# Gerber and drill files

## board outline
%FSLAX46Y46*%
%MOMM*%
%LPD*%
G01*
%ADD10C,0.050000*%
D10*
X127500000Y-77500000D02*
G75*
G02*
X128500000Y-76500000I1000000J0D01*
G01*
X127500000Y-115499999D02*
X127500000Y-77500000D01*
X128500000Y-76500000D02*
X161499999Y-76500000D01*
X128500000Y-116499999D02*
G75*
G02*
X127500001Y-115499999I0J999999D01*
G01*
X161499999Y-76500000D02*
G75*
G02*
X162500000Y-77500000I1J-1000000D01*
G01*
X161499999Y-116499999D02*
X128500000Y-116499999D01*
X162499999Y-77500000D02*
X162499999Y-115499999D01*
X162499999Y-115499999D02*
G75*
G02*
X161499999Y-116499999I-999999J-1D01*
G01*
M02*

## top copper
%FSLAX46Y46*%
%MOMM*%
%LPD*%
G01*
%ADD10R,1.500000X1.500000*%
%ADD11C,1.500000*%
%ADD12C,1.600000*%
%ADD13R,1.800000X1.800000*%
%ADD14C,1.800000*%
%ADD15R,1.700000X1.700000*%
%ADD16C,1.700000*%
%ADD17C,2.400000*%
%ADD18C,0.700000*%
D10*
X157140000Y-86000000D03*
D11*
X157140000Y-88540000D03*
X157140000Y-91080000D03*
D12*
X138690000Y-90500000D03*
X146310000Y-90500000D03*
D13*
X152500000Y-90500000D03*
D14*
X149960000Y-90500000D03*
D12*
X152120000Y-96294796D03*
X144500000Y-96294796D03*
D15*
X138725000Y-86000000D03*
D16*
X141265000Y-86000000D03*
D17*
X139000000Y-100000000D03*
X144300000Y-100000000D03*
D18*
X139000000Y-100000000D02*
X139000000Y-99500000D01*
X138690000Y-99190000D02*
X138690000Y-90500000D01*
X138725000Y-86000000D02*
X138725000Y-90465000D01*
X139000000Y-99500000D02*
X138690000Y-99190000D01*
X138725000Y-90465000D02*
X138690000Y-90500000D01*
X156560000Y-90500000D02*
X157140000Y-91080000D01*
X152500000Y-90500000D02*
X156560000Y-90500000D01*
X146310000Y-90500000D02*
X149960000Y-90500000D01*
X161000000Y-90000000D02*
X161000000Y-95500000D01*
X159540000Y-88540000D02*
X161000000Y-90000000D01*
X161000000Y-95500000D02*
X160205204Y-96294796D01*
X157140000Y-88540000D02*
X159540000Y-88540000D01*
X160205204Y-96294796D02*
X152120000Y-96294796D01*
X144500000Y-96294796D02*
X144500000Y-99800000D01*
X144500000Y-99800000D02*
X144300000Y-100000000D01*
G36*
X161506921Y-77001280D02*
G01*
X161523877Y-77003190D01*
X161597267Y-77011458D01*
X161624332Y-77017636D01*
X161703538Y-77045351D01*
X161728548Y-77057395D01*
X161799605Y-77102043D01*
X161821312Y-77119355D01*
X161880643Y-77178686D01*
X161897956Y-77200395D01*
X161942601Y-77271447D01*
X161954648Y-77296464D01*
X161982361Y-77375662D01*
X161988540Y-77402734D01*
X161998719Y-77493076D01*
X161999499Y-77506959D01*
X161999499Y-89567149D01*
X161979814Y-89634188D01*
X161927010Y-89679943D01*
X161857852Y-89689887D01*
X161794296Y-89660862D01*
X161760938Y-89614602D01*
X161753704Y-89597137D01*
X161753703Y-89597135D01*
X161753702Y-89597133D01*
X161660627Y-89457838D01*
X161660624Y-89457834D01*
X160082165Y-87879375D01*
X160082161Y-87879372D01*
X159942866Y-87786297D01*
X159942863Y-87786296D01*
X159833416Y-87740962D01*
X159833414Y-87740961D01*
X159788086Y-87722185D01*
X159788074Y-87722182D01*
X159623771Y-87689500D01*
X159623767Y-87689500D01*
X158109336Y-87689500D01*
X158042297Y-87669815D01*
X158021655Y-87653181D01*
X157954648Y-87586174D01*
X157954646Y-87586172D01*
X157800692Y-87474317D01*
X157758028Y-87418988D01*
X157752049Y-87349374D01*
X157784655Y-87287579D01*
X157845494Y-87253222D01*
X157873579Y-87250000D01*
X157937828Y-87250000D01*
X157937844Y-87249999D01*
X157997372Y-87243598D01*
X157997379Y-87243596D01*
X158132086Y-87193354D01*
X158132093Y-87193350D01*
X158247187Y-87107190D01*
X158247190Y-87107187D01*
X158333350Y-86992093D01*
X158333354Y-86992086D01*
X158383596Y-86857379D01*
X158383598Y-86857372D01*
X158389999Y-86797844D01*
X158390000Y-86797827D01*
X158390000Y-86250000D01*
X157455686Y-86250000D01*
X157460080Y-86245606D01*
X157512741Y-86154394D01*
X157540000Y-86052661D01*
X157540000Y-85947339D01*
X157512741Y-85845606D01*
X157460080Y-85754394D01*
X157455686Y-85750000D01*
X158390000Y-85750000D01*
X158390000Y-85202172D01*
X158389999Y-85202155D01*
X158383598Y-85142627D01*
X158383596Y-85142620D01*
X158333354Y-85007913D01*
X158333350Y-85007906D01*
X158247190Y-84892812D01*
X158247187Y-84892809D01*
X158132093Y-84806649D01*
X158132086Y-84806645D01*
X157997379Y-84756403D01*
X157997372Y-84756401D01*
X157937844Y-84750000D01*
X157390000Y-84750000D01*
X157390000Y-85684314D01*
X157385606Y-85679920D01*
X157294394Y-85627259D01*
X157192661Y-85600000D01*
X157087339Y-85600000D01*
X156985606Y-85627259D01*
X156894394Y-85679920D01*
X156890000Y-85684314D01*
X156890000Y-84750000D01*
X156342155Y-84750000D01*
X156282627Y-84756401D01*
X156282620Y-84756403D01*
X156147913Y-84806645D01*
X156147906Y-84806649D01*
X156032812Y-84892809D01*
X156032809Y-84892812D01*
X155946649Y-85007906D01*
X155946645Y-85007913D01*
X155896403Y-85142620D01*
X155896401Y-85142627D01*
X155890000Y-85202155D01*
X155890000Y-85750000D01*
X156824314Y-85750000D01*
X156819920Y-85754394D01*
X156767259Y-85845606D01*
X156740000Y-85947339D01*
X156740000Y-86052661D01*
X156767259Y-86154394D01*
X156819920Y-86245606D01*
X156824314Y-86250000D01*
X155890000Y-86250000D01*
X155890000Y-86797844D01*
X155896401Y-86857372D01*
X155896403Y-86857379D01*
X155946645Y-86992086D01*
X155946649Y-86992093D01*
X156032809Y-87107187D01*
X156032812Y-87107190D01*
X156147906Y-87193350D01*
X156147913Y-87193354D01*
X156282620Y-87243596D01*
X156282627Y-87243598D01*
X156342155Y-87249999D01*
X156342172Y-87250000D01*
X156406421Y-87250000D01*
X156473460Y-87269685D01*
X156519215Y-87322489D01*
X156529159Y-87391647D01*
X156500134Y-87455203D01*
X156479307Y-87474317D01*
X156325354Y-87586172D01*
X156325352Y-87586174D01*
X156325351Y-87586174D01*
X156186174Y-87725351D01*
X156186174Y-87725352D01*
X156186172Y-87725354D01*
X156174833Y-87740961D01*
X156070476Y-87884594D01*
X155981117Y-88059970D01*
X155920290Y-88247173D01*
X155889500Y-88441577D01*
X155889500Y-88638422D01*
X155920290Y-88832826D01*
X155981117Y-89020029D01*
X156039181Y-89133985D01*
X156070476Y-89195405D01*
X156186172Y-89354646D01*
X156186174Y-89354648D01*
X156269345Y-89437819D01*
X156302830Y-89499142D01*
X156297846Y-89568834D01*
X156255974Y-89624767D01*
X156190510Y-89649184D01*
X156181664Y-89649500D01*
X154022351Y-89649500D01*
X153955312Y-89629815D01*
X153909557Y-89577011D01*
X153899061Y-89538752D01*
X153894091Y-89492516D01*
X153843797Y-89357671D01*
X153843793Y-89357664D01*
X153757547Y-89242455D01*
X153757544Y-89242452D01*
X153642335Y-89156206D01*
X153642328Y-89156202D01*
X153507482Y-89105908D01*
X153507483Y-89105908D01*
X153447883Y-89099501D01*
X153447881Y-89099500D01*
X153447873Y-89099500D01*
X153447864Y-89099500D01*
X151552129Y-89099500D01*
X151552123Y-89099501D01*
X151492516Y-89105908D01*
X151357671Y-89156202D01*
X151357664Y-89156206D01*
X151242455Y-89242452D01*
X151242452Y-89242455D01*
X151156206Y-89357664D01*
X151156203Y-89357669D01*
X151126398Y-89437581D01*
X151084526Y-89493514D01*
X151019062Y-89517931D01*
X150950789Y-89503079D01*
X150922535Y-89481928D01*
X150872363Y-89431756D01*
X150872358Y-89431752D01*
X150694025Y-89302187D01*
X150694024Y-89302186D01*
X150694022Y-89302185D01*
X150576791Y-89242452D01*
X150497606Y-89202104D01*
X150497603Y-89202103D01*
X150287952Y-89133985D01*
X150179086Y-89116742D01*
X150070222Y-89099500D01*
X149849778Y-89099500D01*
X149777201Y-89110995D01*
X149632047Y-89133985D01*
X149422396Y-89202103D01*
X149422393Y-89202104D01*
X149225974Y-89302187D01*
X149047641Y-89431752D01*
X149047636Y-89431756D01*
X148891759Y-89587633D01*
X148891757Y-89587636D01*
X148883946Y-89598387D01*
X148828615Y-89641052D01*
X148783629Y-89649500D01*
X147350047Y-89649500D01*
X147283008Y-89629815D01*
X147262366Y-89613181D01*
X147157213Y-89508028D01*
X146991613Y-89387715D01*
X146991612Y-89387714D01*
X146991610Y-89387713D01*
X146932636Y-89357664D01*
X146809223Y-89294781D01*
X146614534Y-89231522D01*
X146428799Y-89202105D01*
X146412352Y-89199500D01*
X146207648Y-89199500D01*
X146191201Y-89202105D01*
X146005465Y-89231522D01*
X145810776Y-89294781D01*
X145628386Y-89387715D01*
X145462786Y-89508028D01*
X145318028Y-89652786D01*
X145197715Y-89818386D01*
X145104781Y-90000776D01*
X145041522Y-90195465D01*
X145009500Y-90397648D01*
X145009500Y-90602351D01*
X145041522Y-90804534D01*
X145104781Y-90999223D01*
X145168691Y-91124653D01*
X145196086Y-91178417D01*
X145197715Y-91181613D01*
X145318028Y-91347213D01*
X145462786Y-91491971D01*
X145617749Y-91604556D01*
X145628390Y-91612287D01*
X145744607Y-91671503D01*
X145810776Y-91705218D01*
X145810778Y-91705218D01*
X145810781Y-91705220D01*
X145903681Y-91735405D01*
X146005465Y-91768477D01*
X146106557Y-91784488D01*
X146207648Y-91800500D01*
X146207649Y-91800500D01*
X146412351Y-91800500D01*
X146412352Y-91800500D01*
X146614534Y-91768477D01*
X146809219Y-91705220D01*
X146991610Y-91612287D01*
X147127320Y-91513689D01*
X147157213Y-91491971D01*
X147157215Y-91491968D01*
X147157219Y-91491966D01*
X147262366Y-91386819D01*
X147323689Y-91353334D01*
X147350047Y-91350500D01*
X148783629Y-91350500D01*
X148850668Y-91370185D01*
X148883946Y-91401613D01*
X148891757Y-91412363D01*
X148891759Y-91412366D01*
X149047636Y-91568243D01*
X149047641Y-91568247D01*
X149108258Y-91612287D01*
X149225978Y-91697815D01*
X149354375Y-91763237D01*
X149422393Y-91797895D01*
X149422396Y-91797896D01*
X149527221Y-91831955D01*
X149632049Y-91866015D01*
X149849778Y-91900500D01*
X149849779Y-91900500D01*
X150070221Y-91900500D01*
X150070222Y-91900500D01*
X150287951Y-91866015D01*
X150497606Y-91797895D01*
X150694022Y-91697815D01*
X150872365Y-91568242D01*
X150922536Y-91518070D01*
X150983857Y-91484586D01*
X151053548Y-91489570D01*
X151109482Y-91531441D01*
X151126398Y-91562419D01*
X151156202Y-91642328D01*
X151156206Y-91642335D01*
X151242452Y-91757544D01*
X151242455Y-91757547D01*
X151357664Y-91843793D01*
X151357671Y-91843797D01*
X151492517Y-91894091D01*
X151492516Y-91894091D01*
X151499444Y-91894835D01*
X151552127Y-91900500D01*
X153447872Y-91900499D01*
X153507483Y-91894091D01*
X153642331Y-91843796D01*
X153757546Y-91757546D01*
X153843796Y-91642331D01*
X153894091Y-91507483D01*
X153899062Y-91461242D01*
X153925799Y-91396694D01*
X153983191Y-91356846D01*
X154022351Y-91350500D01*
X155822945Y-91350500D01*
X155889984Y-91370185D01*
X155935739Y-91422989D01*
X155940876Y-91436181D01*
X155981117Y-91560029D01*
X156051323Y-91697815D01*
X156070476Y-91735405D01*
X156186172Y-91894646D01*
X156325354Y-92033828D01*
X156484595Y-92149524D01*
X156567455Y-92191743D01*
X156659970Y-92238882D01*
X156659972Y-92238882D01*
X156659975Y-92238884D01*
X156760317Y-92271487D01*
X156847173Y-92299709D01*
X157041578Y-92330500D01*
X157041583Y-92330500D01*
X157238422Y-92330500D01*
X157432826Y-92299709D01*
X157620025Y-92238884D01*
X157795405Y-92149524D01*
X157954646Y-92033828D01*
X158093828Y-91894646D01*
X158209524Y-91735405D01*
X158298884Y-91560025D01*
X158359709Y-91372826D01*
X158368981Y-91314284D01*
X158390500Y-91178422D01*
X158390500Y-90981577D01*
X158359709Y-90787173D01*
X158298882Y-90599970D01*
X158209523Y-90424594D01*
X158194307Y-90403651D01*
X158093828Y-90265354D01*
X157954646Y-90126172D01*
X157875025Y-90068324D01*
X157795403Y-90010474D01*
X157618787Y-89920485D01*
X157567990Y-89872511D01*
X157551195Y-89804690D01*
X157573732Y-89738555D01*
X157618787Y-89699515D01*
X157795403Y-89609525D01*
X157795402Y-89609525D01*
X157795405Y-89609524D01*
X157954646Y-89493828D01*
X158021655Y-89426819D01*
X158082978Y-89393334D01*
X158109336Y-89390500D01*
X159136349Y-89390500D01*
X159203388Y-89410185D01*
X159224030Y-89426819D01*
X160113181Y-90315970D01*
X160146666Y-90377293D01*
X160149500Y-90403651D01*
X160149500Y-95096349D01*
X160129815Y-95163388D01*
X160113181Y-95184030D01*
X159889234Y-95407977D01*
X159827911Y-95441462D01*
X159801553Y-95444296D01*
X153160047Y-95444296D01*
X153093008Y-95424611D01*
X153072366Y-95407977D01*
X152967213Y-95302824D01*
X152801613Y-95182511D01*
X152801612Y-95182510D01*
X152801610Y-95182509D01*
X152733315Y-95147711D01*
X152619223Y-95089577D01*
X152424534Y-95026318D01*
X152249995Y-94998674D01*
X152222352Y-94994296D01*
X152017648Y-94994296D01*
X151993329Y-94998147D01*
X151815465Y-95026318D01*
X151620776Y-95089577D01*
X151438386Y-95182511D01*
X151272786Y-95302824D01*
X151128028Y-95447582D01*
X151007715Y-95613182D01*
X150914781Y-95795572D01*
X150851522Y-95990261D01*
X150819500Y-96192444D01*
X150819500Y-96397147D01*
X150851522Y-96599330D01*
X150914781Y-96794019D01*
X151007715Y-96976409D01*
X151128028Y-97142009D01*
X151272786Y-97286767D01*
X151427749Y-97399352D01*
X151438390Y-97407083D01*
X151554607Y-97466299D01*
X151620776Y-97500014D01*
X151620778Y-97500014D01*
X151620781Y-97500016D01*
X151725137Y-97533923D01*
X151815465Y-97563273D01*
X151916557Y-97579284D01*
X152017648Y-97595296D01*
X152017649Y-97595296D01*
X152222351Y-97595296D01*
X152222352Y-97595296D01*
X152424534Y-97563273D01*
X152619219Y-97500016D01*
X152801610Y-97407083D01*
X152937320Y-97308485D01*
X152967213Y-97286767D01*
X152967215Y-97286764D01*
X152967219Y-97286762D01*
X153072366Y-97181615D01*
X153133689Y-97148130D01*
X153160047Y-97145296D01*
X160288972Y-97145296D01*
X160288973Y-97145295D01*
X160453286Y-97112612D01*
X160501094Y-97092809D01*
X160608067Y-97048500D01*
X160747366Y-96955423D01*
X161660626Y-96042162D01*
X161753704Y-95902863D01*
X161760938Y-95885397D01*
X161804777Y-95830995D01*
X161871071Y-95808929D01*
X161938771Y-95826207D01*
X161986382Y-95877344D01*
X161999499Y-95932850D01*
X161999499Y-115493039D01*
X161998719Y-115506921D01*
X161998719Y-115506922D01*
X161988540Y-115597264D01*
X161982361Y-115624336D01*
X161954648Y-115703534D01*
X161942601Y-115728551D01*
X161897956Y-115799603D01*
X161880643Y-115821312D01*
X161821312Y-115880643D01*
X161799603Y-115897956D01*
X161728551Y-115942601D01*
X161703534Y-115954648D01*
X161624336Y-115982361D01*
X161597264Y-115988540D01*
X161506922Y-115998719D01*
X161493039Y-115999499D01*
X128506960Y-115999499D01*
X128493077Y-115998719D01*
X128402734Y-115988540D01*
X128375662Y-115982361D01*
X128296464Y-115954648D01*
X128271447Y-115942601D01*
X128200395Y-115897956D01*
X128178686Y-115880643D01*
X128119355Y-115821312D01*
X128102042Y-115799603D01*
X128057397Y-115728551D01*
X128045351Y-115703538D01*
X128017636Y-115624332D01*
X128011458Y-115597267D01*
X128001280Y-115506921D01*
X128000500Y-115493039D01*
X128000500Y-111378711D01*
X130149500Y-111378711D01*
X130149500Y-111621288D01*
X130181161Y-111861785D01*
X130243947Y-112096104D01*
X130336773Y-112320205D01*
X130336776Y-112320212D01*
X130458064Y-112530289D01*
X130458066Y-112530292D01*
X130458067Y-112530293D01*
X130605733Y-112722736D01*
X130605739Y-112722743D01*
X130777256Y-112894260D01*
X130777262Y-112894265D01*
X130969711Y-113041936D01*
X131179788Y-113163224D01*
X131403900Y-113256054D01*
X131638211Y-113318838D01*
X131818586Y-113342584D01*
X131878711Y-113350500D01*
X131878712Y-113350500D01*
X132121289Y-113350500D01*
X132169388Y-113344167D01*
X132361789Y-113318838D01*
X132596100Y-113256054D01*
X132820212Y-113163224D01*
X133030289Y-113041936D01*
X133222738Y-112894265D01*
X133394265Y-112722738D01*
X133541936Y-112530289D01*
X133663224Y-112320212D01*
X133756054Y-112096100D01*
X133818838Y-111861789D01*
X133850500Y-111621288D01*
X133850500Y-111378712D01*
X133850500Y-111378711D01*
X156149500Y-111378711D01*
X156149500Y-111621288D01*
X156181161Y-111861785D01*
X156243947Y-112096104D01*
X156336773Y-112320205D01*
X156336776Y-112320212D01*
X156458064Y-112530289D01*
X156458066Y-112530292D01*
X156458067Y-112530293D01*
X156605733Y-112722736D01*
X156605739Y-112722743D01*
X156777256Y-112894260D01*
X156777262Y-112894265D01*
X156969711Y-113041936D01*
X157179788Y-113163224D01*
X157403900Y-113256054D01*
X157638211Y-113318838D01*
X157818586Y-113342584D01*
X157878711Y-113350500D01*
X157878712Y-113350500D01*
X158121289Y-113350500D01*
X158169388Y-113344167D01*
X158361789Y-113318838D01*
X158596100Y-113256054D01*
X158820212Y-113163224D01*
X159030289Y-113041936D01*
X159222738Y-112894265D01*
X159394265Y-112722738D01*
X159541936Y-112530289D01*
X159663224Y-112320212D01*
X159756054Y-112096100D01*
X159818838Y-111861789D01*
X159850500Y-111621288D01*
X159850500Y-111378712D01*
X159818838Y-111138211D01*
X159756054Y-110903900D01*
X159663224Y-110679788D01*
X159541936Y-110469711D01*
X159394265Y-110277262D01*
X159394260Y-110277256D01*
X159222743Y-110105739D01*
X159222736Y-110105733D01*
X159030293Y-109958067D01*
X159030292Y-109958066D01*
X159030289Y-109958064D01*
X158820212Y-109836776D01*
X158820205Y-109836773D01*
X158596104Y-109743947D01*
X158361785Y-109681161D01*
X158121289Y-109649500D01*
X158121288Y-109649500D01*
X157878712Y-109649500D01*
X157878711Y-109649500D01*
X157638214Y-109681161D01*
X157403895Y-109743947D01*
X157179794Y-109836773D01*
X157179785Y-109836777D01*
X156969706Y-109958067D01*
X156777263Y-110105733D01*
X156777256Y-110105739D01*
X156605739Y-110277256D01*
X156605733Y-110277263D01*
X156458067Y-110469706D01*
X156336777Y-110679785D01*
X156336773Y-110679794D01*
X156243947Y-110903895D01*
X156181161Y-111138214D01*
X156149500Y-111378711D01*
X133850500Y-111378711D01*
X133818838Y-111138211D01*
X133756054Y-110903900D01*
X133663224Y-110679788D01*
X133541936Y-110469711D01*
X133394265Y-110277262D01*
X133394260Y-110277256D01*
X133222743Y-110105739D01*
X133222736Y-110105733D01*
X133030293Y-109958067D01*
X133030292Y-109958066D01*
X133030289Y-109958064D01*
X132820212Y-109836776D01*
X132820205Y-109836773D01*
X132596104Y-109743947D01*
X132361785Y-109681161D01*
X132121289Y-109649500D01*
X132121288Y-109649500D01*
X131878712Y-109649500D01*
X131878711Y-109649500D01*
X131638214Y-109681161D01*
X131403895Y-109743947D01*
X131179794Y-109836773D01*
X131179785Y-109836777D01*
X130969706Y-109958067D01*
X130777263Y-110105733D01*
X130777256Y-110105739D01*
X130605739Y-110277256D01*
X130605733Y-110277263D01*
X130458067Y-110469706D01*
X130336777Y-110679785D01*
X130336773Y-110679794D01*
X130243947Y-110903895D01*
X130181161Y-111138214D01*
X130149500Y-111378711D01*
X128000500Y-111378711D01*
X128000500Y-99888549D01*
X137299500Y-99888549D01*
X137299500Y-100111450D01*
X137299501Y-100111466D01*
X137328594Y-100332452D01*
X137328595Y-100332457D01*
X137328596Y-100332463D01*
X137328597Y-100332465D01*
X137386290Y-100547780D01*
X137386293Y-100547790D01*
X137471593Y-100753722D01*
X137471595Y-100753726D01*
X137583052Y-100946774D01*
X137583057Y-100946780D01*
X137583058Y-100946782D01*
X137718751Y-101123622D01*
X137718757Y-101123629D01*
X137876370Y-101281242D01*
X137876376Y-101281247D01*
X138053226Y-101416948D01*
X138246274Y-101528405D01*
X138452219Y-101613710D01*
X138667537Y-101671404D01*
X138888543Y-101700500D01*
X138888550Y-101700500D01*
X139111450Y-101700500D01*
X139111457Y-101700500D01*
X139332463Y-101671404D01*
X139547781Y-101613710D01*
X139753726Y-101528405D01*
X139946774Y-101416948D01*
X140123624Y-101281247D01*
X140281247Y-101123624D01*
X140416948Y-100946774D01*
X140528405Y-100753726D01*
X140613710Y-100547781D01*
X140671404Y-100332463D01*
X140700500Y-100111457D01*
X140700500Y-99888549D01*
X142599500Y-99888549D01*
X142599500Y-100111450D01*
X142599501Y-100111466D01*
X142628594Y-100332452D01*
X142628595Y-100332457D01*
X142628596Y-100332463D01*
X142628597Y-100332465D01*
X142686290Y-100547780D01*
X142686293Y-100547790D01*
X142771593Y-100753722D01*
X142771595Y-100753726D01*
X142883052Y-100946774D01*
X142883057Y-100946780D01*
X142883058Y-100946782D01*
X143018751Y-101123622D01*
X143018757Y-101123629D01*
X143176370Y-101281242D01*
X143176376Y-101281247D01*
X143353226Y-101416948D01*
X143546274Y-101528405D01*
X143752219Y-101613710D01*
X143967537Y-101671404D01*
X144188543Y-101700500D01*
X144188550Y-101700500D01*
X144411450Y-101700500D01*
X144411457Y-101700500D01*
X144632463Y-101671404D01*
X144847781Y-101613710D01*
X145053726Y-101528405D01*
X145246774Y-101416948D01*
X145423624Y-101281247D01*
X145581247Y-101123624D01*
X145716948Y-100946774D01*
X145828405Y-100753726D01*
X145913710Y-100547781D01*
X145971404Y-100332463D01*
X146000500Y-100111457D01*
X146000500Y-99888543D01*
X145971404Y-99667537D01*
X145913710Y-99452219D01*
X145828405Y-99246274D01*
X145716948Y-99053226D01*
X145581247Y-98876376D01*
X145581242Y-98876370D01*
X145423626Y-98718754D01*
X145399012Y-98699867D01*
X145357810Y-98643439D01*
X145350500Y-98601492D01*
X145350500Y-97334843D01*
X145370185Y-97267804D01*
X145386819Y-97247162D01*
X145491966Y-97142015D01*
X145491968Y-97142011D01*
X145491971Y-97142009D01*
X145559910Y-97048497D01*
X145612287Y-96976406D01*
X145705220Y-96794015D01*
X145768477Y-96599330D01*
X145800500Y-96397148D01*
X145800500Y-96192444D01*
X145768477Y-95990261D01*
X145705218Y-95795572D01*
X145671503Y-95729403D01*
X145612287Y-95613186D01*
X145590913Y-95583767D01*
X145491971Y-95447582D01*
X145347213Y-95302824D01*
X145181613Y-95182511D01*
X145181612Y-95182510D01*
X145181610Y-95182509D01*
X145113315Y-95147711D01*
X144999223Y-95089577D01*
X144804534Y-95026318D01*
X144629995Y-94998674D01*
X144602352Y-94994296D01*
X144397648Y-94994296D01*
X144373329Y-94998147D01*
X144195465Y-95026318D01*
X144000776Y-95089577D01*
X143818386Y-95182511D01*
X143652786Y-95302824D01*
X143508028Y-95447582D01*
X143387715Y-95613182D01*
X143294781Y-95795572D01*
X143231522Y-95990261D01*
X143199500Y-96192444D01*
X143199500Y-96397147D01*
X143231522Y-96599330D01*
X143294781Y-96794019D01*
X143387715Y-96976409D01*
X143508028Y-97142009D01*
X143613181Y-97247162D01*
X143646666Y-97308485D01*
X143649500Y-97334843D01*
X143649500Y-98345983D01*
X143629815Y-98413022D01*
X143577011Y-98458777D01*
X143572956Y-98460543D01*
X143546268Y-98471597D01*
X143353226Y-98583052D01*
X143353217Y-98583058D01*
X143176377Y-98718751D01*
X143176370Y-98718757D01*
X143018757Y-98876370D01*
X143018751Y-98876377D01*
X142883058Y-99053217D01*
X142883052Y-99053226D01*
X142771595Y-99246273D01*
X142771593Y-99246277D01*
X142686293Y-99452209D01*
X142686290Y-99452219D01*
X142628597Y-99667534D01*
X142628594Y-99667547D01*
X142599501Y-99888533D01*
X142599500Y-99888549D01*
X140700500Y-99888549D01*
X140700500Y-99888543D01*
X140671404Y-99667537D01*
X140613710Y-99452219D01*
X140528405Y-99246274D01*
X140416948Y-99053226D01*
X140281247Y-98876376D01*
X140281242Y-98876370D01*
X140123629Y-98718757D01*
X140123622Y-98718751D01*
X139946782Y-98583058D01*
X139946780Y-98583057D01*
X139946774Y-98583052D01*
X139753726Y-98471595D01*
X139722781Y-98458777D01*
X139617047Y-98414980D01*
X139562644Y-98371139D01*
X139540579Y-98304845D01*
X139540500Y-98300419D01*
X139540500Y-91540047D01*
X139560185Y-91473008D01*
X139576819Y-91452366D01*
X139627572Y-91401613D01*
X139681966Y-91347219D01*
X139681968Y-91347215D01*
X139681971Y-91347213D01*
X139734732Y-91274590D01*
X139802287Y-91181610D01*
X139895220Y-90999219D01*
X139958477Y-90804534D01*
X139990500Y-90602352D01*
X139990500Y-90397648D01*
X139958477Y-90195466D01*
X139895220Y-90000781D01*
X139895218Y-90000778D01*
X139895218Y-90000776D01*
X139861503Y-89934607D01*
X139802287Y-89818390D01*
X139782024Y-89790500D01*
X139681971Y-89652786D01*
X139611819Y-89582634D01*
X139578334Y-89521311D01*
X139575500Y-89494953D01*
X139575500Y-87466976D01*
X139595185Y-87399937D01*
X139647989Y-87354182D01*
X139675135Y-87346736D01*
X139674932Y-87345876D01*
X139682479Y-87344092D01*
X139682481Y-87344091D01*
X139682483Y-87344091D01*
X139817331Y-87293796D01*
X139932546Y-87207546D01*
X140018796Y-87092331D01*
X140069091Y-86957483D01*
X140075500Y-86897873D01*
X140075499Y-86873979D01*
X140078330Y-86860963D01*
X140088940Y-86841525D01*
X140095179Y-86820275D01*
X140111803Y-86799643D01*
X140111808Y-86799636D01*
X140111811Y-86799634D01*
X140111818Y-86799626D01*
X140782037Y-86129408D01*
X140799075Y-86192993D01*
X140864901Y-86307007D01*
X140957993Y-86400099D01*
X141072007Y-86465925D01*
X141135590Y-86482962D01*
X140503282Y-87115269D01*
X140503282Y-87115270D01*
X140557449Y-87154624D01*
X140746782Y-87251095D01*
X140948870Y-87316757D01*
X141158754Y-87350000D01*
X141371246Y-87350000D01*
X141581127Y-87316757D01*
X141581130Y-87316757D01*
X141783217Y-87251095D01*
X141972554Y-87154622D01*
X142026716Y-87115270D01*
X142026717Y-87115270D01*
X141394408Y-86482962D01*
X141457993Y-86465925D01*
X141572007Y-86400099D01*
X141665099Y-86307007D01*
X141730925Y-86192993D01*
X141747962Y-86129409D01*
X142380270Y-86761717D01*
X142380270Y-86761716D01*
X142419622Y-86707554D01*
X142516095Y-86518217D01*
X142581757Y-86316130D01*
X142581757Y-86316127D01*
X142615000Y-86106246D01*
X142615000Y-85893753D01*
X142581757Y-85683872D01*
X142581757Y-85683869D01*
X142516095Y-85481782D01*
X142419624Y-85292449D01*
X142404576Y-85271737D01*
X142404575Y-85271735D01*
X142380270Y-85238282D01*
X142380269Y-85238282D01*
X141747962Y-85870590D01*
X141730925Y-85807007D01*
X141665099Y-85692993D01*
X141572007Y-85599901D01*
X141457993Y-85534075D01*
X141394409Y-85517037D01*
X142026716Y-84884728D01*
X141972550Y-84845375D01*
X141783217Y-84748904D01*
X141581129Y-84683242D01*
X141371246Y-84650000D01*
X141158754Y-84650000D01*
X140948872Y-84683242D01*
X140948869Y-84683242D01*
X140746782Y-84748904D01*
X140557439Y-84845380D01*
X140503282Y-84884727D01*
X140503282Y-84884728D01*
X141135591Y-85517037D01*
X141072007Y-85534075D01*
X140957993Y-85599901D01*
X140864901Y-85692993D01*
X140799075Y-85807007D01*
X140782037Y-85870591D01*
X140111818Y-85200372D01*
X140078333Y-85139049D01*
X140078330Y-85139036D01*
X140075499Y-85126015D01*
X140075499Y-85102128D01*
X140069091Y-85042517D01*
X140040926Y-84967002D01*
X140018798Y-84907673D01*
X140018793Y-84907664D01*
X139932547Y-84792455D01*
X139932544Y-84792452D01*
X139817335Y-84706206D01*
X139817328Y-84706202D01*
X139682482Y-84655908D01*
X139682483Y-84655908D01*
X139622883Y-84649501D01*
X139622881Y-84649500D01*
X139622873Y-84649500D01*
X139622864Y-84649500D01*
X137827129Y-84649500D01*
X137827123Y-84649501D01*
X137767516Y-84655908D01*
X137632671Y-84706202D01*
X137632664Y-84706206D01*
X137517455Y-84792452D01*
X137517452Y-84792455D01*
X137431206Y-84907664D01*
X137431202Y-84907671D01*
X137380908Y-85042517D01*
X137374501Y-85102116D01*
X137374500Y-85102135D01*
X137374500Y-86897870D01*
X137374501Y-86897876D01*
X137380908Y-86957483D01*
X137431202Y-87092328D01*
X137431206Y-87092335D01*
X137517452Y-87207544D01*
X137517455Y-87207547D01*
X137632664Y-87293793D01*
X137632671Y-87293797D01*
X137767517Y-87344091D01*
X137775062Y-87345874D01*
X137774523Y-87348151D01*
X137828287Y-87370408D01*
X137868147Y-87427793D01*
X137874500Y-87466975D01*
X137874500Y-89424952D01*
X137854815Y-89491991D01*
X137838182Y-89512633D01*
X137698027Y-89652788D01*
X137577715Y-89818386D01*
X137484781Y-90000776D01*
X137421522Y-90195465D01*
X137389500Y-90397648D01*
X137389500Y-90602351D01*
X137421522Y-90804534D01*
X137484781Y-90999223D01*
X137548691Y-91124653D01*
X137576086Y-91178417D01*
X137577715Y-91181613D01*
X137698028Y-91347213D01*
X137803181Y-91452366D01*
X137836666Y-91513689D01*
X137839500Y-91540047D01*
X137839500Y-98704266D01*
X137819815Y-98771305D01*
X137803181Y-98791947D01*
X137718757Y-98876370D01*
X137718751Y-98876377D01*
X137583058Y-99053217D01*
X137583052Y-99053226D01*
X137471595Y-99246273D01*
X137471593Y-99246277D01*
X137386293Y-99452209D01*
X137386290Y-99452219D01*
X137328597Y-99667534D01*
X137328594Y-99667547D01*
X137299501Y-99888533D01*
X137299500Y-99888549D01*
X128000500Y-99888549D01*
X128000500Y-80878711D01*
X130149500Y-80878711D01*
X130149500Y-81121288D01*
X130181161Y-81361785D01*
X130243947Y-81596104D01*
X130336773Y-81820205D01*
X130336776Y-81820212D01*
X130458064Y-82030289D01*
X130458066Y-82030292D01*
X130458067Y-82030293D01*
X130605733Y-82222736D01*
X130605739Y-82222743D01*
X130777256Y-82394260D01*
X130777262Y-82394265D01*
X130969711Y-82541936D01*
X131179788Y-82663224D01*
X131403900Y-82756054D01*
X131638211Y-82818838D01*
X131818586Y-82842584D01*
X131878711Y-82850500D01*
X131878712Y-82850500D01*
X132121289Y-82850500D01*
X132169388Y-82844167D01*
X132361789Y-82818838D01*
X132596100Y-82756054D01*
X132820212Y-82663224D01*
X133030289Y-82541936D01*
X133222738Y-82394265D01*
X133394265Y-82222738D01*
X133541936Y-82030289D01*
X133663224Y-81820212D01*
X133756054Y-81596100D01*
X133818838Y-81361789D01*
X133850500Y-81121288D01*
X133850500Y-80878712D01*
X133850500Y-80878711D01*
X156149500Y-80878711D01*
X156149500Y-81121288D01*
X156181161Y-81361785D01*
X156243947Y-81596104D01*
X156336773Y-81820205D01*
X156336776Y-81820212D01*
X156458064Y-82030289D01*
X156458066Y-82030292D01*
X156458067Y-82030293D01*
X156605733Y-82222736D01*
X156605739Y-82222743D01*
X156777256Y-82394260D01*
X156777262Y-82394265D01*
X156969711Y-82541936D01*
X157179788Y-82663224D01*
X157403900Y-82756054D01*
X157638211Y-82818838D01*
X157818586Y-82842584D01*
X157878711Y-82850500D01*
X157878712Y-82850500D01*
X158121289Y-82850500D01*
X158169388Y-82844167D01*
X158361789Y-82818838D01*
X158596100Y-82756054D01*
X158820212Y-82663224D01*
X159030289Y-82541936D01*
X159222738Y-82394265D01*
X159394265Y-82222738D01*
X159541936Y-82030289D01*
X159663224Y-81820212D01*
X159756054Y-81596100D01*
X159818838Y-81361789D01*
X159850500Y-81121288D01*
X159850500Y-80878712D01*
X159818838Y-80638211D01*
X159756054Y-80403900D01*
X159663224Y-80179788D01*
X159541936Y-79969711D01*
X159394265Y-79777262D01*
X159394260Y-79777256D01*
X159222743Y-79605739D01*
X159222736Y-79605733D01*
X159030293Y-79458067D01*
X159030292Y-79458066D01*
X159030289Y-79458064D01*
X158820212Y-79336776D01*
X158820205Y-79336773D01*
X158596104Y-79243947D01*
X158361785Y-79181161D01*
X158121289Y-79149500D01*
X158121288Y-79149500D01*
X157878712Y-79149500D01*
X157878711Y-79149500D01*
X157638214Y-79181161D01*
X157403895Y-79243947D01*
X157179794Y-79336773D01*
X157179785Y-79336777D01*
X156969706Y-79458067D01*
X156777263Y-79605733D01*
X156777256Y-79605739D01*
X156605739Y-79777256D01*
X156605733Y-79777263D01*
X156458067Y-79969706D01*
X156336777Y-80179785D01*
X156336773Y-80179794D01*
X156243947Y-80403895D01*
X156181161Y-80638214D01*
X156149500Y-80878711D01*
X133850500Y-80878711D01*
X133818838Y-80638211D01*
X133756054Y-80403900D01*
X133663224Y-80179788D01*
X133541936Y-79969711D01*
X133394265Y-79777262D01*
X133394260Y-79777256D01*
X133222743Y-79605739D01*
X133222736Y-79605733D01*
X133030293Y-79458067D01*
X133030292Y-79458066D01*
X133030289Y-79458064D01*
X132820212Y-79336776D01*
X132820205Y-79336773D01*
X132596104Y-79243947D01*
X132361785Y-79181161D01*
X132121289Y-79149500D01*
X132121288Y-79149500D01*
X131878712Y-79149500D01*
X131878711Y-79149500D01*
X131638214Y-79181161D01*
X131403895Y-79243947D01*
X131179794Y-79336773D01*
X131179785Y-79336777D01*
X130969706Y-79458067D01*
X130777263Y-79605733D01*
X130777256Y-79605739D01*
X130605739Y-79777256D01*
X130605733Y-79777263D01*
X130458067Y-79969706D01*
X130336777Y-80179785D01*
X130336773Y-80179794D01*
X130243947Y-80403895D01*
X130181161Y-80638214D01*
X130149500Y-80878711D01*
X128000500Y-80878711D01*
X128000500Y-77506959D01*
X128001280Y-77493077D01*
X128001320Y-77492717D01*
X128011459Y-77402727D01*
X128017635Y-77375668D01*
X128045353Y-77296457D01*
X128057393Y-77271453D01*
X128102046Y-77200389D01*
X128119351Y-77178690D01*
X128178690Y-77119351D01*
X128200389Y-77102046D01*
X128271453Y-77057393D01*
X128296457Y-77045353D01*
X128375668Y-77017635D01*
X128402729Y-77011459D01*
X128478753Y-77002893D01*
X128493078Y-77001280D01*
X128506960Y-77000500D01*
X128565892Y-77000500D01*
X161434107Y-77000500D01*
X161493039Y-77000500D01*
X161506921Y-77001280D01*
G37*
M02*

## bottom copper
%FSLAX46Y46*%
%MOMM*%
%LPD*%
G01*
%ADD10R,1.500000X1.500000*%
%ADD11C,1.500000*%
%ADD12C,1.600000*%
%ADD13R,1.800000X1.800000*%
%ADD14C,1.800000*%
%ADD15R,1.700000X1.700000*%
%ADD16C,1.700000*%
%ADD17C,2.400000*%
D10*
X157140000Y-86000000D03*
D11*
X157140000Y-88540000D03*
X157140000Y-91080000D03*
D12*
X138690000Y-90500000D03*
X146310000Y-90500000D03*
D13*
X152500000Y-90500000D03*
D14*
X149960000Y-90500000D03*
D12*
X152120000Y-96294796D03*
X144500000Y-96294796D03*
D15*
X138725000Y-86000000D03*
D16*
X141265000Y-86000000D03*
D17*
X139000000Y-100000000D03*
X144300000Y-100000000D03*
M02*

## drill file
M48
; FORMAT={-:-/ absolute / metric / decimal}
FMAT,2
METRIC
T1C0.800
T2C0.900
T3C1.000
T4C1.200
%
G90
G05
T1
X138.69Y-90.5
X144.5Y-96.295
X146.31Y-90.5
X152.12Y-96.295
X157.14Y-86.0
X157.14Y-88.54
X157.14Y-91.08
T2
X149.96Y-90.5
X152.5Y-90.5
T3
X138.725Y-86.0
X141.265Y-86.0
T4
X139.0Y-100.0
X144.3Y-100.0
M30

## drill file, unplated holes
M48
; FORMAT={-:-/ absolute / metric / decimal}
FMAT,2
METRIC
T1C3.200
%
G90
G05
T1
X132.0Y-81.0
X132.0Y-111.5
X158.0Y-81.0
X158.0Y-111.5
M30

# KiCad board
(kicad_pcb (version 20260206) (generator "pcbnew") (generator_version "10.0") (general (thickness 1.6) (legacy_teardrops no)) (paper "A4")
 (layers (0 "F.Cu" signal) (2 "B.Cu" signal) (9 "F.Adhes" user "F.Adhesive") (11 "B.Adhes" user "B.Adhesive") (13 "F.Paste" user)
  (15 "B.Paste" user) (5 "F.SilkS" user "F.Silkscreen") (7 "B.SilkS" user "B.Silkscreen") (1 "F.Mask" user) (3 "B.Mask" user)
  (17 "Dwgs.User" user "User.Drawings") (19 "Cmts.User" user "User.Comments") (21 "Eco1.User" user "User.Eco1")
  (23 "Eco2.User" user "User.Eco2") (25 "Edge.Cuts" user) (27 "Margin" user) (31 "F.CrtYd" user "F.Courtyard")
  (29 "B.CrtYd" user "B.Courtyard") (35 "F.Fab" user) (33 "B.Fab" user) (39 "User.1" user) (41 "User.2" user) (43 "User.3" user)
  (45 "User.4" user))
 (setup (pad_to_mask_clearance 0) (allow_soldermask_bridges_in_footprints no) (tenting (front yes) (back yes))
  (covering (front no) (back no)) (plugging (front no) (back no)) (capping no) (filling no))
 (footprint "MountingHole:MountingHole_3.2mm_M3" (layer "F.Cu") (at 132 81)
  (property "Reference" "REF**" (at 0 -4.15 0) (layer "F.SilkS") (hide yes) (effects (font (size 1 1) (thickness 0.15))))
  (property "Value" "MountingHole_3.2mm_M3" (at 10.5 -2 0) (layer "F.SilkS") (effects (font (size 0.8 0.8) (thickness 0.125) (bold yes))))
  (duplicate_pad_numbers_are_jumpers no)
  (pad "" np_thru_hole circle (at 0 0) (size 3.2 3.2) (drill 3.2) (layers "*.Cu" "*.Mask")))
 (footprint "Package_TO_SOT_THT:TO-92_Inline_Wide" (layer "F.Cu") (at 157.14 86 -90)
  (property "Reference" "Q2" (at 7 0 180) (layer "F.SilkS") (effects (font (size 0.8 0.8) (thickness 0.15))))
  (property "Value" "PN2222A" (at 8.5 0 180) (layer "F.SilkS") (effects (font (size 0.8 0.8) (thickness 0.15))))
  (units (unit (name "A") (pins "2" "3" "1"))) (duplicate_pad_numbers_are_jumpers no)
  (pad "1" thru_hole rect (at 0 0 270) (size 1.5 1.5) (drill 0.8) (layers "*.Cu" "*.Mask") (remove_unused_layers no) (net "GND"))
  (pad "2" thru_hole circle (at 2.54 0 270) (size 1.5 1.5) (drill 0.8) (layers "*.Cu" "*.Mask") (remove_unused_layers no) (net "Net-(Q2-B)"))
  (pad "3" thru_hole circle (at 5.08 0 270) (size 1.5 1.5) (drill 0.8) (layers "*.Cu" "*.Mask") (remove_unused_layers no) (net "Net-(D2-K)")))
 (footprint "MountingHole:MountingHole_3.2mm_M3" (layer "F.Cu") (at 158 81)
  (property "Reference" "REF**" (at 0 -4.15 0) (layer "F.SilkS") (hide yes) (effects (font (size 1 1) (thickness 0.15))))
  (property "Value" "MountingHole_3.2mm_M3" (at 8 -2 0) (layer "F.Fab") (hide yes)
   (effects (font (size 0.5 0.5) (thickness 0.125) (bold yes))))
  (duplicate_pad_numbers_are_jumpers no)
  (pad "" np_thru_hole circle (at 0 0) (size 3.2 3.2) (drill 3.2) (layers "*.Cu" "*.Mask")))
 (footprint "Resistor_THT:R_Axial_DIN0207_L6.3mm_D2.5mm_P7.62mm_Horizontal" (layer "F.Cu") (at 138.69 90.5)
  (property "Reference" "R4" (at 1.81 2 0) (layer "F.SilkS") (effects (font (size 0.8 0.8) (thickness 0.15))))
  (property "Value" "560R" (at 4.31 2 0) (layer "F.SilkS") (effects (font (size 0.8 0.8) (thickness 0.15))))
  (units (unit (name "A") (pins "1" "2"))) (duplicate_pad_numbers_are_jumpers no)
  (pad "1" thru_hole circle (at 0 0) (size 1.6 1.6) (drill 0.8) (layers "*.Cu" "*.Mask") (remove_unused_layers no) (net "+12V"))
  (pad "2" thru_hole circle (at 7.62 0) (size 1.6 1.6) (drill 0.8) (layers "*.Cu" "*.Mask") (remove_unused_layers no) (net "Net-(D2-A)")))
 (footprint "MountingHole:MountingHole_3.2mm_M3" (layer "F.Cu") (at 158 111.5)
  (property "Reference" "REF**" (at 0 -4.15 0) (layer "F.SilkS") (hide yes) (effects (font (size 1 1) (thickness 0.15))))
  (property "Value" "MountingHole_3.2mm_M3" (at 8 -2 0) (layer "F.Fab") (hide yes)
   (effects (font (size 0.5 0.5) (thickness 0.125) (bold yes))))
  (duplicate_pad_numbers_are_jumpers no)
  (pad "" np_thru_hole circle (at 0 0) (size 3.2 3.2) (drill 3.2) (layers "*.Cu" "*.Mask")))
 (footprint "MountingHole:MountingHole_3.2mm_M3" (layer "F.Cu") (at 132 111.5)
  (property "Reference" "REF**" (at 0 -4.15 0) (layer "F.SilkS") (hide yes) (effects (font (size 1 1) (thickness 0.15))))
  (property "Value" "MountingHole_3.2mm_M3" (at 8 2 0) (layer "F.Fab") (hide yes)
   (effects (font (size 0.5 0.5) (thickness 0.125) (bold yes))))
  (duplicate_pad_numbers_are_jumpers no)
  (pad "" np_thru_hole circle (at 0 0) (size 3.2 3.2) (drill 3.2) (layers "*.Cu" "*.Mask")))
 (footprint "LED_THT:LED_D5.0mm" (layer "F.Cu") (at 152.5 90.5 180)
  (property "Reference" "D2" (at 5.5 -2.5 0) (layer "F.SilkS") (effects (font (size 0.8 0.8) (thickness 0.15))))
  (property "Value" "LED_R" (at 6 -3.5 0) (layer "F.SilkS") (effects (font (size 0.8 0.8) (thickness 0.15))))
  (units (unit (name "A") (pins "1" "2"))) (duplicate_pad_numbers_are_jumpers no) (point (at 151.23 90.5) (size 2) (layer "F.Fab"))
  (pad "1" thru_hole rect (at 0 0 180) (size 1.8 1.8) (drill 0.9) (layers "*.Cu" "*.Mask") (remove_unused_layers no) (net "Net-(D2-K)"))
  (pad "2" thru_hole circle (at 2.54 0 180) (size 1.8 1.8) (drill 0.9) (layers "*.Cu" "*.Mask") (remove_unused_layers no) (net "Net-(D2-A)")))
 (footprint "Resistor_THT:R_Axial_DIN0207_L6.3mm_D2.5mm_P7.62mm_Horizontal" (layer "F.Cu") (at 152.12 96.294796 180)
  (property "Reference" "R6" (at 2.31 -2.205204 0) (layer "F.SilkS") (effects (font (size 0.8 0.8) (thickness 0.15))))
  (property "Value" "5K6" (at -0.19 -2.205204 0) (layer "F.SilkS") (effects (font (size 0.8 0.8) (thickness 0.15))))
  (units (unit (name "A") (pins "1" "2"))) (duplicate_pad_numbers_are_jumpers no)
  (pad "1" thru_hole circle (at 0 0 180) (size 1.6 1.6) (drill 0.8) (layers "*.Cu" "*.Mask") (remove_unused_layers no) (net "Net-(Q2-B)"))
  (pad "2" thru_hole circle (at 7.62 0 180) (size 1.6 1.6) (drill 0.8) (layers "*.Cu" "*.Mask") (remove_unused_layers no)
   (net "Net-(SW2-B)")))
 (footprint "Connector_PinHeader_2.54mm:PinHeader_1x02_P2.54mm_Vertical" (layer "F.Cu") (at 138.725 86 90)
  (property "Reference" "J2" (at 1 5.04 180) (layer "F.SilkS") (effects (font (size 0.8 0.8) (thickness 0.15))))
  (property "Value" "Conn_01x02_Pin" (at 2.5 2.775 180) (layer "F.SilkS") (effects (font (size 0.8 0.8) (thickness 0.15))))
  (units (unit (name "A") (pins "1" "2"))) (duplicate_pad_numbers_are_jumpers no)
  (pad "1" thru_hole rect (at 0 0 90) (size 1.7 1.7) (drill 1) (layers "*.Cu" "*.Mask") (remove_unused_layers no) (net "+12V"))
  (pad "2" thru_hole circle (at 0 2.54 90) (size 1.7 1.7) (drill 1) (layers "*.Cu" "*.Mask") (remove_unused_layers no) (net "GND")))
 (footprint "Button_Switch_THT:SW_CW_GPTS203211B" (layer "B.Cu") (at 139 100 -90)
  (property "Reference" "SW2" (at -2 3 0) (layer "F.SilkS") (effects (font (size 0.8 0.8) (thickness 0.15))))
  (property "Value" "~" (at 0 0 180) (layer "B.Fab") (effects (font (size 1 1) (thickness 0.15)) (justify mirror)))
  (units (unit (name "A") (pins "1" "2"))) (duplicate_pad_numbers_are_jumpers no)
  (pad "1" thru_hole circle (at 0 0 270) (size 2.4 2.4) (drill 1.2) (layers "*.Cu" "*.Mask") (remove_unused_layers no) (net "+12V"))
  (pad "2" thru_hole circle (at 0 -5.3 270) (size 2.4 2.4) (drill 1.2) (layers "*.Cu" "*.Mask") (remove_unused_layers no)
   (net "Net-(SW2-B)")))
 (gr_arc (start 127.5 77.5) (mid 127.792893 76.792893) (end 128.5 76.5) (stroke (width 0.05) (type default)) (layer "Edge.Cuts"))
 (gr_line (start 127.5 115.499999) (end 127.5 77.5) (stroke (width 0.05) (type default)) (layer "Edge.Cuts"))
 (gr_line (start 128.5 76.5) (end 161.499999 76.5) (stroke (width 0.05) (type default)) (layer "Edge.Cuts"))
 (gr_arc (start 128.5 116.499999) (mid 127.792893 116.207106) (end 127.5 115.499999) (stroke (width 0.05) (type default))
  (layer "Edge.Cuts"))
 (gr_arc (start 161.499999 76.5) (mid 162.207106 76.792893) (end 162.499999 77.5) (stroke (width 0.05) (type default)) (layer "Edge.Cuts"))
 (gr_line (start 161.499999 116.499999) (end 128.5 116.499999) (stroke (width 0.05) (type default)) (layer "Edge.Cuts"))
 (gr_line (start 162.499999 77.5) (end 162.499999 115.499999) (stroke (width 0.05) (type default)) (layer "Edge.Cuts"))
 (gr_arc (start 162.499999 115.499999) (mid 162.207106 116.207106) (end 161.499999 116.499999) (stroke (width 0.05) (type default))
  (layer "Edge.Cuts"))
 (segment (start 139 100) (end 139 99.5) (width 0.7) (layer "F.Cu") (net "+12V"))
 (segment (start 138.69 99.19) (end 138.69 90.5) (width 0.7) (layer "F.Cu") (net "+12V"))
 (segment (start 138.725 86) (end 138.725 90.465) (width 0.7) (layer "F.Cu") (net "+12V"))
 (segment (start 139 99.5) (end 138.69 99.19) (width 0.7) (layer "F.Cu") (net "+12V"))
 (segment (start 138.725 90.465) (end 138.69 90.5) (width 0.7) (layer "F.Cu") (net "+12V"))
 (segment (start 156.56 90.5) (end 157.14 91.08) (width 0.7) (layer "F.Cu") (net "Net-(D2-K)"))
 (segment (start 152.5 90.5) (end 156.56 90.5) (width 0.7) (layer "F.Cu") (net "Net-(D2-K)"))
 (segment (start 146.31 90.5) (end 149.96 90.5) (width 0.7) (layer "F.Cu") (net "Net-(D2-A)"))
 (segment (start 161 90) (end 161 95.5) (width 0.7) (layer "F.Cu") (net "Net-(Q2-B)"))
 (segment (start 159.54 88.54) (end 161 90) (width 0.7) (layer "F.Cu") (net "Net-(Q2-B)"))
 (segment (start 161 95.5) (end 160.205204 96.294796) (width 0.7) (layer "F.Cu") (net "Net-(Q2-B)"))
 (segment (start 157.14 88.54) (end 159.54 88.54) (width 0.7) (layer "F.Cu") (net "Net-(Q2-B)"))
 (segment (start 160.205204 96.294796) (end 152.12 96.294796) (width 0.7) (layer "F.Cu") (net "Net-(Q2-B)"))
 (segment (start 144.5 96.294796) (end 144.5 99.8) (width 0.7) (layer "F.Cu") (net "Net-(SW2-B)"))
 (segment (start 144.5 99.8) (end 144.3 100) (width 0.7) (layer "F.Cu") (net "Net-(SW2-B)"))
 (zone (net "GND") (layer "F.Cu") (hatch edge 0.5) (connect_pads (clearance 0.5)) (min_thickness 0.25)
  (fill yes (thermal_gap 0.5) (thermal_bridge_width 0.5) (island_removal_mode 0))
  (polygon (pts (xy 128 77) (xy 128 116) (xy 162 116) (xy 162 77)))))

